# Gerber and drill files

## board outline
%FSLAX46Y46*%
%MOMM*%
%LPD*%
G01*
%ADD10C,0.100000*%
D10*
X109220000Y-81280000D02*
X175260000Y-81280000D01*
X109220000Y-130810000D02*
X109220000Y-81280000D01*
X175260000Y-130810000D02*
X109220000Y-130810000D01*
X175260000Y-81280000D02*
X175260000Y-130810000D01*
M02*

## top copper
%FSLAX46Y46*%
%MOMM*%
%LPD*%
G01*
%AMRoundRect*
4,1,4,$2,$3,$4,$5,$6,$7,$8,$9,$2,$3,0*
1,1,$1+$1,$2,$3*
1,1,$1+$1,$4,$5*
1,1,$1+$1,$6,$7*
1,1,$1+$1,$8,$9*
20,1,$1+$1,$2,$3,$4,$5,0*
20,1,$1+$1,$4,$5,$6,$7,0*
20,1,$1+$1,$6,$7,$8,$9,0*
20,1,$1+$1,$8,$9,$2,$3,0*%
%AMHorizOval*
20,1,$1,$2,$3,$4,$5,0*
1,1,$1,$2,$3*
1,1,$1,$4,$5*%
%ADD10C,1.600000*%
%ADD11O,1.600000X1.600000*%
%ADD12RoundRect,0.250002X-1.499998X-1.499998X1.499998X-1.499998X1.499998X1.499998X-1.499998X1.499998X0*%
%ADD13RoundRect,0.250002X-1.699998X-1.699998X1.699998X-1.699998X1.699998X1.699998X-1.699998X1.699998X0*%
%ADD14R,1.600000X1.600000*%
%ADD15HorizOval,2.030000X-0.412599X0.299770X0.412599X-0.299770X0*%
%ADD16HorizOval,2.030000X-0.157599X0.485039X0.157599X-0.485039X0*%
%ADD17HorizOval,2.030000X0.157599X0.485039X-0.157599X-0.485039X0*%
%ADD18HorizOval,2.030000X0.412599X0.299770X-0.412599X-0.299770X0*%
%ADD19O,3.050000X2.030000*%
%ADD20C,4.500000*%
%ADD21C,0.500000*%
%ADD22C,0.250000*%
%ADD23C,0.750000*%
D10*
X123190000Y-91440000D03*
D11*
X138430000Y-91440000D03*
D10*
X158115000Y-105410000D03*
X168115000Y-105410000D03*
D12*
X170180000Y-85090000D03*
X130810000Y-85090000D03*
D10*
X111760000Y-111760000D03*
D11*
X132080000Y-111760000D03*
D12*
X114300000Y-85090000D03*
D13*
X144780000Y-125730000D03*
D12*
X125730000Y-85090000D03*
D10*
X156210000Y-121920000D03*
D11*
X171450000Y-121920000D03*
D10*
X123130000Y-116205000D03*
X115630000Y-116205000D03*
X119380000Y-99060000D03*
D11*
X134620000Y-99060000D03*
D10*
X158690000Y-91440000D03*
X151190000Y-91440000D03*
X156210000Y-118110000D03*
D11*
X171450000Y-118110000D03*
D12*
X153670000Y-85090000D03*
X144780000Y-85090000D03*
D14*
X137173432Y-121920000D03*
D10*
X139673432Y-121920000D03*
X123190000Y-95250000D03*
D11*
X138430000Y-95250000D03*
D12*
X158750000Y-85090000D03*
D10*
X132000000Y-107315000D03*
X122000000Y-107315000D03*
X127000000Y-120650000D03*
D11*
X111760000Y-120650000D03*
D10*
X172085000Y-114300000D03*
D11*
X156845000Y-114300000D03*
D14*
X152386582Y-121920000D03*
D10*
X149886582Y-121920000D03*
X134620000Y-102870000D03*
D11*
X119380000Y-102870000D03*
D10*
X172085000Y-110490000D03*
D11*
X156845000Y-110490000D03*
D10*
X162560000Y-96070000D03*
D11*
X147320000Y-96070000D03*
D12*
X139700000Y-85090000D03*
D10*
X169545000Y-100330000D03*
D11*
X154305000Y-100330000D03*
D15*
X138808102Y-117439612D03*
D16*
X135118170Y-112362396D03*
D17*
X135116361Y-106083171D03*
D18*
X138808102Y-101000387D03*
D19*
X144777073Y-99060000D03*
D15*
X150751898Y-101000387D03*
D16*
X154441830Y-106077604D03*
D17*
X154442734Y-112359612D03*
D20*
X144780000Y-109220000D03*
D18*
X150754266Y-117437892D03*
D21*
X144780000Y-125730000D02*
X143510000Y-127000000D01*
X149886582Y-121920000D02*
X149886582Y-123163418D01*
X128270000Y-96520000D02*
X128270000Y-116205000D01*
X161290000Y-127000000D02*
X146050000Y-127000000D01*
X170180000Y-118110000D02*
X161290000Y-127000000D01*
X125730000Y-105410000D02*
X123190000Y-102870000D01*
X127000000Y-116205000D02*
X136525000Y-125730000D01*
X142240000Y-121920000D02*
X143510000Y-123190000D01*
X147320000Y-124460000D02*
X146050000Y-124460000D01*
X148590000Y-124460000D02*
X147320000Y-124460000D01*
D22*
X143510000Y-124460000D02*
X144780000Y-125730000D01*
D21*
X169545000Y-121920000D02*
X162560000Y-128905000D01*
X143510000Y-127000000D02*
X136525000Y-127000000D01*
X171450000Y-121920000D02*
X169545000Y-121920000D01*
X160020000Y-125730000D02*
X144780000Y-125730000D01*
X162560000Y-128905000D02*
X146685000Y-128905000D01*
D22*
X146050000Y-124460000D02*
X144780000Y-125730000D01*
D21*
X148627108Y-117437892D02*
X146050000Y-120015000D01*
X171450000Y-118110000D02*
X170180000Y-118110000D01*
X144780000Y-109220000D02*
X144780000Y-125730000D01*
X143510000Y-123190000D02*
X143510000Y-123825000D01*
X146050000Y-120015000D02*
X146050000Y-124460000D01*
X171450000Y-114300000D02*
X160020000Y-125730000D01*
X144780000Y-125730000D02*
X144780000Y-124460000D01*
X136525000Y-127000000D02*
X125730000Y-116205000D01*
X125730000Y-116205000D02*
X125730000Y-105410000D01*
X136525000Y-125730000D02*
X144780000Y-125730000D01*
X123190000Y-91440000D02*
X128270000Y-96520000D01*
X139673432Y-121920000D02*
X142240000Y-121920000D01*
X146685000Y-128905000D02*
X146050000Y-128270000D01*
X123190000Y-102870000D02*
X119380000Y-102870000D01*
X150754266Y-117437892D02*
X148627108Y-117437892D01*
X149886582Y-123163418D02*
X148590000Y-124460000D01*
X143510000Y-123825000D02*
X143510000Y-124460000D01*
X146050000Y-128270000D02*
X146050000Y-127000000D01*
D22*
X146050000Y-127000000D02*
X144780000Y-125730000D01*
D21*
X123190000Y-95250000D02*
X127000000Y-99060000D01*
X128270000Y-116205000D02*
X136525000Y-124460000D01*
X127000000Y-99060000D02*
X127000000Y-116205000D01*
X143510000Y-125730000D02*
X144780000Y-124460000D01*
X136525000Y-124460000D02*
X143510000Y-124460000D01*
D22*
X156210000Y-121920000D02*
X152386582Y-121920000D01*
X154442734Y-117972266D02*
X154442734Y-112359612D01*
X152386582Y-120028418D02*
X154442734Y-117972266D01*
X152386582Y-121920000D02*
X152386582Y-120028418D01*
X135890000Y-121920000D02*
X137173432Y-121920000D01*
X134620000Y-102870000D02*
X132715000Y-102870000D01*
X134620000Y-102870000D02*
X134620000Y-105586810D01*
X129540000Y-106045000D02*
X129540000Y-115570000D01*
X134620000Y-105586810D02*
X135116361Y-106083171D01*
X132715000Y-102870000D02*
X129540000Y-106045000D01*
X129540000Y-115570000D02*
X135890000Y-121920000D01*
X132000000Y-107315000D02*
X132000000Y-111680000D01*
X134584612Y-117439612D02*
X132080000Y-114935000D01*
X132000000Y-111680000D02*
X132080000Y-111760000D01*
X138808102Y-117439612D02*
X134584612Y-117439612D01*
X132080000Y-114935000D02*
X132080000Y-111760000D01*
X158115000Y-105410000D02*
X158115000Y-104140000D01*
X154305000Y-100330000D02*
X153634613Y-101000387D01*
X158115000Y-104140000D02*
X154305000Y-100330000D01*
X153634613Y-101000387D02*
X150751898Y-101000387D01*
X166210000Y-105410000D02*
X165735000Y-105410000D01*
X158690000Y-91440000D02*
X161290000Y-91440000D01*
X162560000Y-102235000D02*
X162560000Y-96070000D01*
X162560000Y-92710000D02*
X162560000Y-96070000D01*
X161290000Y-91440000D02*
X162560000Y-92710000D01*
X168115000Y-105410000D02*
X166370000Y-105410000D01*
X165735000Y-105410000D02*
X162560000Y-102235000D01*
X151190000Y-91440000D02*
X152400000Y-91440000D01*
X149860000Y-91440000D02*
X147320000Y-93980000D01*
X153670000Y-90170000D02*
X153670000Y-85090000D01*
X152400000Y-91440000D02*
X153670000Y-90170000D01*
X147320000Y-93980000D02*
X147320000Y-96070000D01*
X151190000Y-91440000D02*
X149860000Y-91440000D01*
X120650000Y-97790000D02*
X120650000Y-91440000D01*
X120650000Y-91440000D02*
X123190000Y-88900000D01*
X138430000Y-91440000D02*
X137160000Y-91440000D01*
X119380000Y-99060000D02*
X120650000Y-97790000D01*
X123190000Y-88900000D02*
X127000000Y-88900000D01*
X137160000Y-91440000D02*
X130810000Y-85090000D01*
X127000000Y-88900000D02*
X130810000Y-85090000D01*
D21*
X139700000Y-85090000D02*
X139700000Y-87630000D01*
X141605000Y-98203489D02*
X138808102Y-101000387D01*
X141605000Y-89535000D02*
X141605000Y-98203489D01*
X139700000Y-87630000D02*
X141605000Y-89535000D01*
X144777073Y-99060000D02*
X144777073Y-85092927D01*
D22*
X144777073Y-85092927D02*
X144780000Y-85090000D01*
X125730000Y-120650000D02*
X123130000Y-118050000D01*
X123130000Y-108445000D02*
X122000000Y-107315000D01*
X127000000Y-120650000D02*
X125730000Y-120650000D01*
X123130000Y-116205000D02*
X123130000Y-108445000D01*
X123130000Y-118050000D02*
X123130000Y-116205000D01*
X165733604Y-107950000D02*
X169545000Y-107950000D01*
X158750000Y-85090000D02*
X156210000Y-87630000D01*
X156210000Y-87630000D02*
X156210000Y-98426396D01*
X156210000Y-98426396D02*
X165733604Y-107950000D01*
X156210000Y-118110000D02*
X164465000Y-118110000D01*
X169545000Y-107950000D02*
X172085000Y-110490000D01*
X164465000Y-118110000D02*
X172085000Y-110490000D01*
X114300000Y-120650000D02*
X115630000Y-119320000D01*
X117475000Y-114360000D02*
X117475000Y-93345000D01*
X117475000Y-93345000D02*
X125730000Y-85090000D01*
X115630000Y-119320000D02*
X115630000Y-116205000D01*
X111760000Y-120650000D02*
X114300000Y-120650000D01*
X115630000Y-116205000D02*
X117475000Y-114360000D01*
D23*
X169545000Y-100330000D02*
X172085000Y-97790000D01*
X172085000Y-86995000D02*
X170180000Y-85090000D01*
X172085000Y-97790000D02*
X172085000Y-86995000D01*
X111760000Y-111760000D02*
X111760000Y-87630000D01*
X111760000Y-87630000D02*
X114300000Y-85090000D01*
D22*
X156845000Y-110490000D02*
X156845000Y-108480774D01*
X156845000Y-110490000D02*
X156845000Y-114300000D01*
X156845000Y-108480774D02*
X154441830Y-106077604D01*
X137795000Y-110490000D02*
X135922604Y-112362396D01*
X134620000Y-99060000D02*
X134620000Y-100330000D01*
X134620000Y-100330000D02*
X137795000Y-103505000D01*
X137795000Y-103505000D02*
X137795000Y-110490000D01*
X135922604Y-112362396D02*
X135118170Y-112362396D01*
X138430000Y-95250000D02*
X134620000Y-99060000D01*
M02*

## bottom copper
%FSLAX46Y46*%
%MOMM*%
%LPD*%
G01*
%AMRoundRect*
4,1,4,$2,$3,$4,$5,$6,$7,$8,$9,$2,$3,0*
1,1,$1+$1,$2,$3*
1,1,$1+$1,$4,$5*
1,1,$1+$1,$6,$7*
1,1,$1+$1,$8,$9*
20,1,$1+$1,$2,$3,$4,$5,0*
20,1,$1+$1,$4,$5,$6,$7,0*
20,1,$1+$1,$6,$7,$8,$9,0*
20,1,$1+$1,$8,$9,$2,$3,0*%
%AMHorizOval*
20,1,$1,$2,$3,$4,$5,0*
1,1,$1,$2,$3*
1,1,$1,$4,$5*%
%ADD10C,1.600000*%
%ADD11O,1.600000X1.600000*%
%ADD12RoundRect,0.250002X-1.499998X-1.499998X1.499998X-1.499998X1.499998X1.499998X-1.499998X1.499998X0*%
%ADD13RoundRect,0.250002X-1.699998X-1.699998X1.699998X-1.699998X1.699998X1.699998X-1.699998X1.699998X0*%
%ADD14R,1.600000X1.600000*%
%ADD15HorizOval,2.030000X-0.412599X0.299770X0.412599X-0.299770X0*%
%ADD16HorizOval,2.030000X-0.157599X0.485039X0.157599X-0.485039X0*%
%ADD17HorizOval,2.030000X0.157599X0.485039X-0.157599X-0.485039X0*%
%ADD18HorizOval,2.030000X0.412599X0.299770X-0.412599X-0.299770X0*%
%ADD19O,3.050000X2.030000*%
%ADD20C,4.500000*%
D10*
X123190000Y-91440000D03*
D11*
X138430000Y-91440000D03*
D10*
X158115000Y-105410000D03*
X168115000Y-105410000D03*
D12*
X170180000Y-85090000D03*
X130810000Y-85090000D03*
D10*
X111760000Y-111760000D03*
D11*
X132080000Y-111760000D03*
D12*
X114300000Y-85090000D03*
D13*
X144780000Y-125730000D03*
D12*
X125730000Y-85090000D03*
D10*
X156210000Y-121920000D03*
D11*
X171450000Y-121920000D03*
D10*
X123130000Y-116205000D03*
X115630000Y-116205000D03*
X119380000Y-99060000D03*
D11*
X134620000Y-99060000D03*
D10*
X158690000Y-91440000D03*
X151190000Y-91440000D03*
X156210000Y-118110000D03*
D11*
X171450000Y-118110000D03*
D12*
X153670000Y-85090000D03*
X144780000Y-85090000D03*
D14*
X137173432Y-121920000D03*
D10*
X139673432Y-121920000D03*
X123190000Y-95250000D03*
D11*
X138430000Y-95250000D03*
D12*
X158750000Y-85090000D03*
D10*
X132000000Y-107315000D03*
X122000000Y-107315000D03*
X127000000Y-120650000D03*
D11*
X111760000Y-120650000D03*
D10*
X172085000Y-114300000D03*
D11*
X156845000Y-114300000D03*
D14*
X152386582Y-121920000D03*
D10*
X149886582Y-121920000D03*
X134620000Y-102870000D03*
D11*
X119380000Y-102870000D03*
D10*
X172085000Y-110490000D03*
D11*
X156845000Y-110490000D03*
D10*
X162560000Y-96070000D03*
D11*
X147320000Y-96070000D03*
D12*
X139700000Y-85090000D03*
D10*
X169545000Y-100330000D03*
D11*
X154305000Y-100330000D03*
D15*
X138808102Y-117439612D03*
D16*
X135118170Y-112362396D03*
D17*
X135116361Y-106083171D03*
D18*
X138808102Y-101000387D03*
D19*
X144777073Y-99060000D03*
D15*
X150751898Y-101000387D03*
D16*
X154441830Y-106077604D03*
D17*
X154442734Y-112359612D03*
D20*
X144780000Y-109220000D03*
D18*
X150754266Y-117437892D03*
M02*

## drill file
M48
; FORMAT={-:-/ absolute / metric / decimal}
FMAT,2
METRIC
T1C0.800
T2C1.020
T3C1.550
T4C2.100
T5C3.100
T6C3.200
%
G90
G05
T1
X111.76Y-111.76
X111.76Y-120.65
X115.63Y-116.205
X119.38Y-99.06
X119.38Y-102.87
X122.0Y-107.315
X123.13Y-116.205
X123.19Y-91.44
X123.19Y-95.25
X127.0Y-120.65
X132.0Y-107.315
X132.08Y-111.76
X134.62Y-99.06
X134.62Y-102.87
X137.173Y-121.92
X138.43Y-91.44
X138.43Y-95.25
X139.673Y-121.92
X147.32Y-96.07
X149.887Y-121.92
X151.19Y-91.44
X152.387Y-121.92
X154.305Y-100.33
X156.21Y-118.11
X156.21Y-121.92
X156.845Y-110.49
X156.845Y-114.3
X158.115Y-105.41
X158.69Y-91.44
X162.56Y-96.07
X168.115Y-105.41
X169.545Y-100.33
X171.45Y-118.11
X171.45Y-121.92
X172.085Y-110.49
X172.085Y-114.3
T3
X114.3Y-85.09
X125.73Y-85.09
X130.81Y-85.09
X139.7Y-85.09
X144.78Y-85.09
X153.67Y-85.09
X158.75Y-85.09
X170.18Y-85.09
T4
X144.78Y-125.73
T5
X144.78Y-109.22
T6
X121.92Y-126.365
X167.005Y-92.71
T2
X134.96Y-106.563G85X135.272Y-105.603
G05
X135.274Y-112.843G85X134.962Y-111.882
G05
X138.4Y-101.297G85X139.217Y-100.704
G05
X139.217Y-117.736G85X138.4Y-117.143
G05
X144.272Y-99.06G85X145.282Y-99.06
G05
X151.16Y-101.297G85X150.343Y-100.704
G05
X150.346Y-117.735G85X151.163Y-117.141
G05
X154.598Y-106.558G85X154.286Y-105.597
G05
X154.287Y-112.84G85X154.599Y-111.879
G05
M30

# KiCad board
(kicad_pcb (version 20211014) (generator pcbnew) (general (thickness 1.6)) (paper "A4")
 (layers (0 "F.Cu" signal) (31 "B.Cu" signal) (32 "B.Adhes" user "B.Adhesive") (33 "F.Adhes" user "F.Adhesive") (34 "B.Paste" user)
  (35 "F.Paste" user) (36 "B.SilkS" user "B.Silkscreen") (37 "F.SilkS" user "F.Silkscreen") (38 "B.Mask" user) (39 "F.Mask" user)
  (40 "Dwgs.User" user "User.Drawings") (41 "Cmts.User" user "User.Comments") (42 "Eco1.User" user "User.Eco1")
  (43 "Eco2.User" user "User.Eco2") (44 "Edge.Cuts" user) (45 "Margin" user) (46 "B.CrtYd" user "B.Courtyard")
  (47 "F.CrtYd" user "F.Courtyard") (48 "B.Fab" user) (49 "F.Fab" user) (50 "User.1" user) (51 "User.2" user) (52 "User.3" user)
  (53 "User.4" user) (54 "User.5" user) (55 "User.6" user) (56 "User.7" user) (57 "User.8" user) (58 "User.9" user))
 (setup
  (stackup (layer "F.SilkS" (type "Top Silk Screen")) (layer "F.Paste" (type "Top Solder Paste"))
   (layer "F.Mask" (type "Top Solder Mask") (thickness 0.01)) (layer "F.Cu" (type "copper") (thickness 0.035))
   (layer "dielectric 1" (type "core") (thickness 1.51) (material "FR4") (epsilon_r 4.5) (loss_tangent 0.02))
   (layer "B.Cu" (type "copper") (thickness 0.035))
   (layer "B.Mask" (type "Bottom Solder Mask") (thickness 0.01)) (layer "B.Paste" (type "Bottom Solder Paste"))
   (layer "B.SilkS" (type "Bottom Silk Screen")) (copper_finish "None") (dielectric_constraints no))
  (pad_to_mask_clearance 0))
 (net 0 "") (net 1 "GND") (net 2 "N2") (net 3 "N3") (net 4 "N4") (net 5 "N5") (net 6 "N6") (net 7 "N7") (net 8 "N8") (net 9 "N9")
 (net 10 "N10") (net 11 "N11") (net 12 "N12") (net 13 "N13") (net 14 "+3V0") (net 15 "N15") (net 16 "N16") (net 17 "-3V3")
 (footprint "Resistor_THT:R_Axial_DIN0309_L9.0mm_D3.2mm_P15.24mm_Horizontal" (layer "F.Cu") (at 123.19 91.44)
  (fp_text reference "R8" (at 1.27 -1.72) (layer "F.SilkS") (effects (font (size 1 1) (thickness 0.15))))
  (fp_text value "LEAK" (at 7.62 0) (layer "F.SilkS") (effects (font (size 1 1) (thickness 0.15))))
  (pad "1" thru_hole circle (at 0 0) (size 1.6 1.6) (drill 0.8) (layers *.Cu *.Mask) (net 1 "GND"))
  (pad "2" thru_hole oval (at 15.24 0) (size 1.6 1.6) (drill 0.8) (layers *.Cu *.Mask) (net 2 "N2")))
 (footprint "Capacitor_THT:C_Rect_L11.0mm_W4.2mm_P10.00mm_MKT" (layer "F.Cu") (at 158.115 105.41)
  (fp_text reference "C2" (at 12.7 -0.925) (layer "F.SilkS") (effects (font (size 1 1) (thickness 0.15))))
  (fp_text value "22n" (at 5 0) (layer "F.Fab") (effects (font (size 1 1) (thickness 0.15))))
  (pad "1" thru_hole circle (at 0 0) (size 1.6 1.6) (drill 0.8) (layers *.Cu *.Mask) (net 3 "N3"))
  (pad "2" thru_hole circle (at 10 0) (size 1.6 1.6) (drill 0.8) (layers *.Cu *.Mask) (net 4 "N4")))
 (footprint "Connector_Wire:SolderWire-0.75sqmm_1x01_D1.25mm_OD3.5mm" (layer "F.Cu") (at 170.18 85.09)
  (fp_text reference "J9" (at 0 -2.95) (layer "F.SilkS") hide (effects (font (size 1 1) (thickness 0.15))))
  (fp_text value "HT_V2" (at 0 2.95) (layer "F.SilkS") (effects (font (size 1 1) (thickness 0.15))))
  (pad "1" thru_hole roundrect (at 0 0) (size 3.5 3.5) (drill 1.55) (layers *.Cu *.Mask) (roundrect_rratio 0.07142914286) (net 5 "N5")))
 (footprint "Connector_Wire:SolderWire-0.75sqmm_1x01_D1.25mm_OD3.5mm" (layer "F.Cu") (at 130.81 85.09)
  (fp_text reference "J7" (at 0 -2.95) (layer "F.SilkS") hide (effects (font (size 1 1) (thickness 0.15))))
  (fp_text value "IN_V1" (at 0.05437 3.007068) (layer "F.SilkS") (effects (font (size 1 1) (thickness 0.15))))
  (pad "1" thru_hole roundrect (at 0 0) (size 3.5 3.5) (drill 1.55) (layers *.Cu *.Mask) (roundrect_rratio 0.07142914286) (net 2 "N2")))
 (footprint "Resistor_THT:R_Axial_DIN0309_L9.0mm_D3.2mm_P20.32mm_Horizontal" (layer "F.Cu") (at 111.76 111.76)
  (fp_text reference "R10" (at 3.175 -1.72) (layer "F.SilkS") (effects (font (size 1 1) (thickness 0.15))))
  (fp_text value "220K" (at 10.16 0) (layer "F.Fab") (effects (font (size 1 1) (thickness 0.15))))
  (pad "1" thru_hole circle (at 0 0) (size 1.6 1.6) (drill 0.8) (layers *.Cu *.Mask) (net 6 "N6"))
  (pad "2" thru_hole oval (at 20.32 0) (size 1.6 1.6) (drill 0.8) (layers *.Cu *.Mask) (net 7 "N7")))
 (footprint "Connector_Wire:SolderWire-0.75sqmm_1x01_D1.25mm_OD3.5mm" (layer "F.Cu") (at 114.3 85.09)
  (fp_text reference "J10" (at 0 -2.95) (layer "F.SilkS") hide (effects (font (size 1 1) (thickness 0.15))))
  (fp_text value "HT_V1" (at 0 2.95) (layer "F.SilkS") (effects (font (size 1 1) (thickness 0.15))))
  (pad "1" thru_hole roundrect (at 0 0) (size 3.5 3.5) (drill 1.55) (layers *.Cu *.Mask) (roundrect_rratio 0.07142914286) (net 6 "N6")))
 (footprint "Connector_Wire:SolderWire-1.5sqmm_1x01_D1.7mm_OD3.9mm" (layer "F.Cu") (at 144.78 125.73)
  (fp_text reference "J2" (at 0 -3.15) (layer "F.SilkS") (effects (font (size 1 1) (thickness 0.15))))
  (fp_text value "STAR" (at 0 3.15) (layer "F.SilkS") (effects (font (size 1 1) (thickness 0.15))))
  (pad "1" thru_hole roundrect (at 0 0) (size 3.9 3.9) (drill 2.1) (layers *.Cu *.Mask) (roundrect_rratio 0.06410307692) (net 1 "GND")))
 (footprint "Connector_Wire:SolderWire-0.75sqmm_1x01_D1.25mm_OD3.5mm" (layer "F.Cu") (at 125.73 85.09)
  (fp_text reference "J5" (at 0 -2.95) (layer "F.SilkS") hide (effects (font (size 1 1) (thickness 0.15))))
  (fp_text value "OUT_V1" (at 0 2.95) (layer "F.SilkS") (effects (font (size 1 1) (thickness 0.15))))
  (pad "1" thru_hole roundrect (at 0 0) (size 3.5 3.5) (drill 1.55) (layers *.Cu *.Mask) (roundrect_rratio 0.07142914286) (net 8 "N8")))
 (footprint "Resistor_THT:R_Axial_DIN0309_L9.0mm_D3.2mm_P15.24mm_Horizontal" (layer "F.Cu") (at 156.21 121.92)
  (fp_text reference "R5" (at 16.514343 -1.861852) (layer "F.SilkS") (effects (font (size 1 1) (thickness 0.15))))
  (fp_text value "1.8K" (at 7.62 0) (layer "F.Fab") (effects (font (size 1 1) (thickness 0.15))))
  (pad "1" thru_hole circle (at 0 0) (size 1.6 1.6) (drill 0.8) (layers *.Cu *.Mask) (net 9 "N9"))
  (pad "2" thru_hole oval (at 15.24 0) (size 1.6 1.6) (drill 0.8) (layers *.Cu *.Mask) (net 1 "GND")))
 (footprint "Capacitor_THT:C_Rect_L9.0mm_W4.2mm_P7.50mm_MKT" (layer "F.Cu") (at 123.13 116.205 180)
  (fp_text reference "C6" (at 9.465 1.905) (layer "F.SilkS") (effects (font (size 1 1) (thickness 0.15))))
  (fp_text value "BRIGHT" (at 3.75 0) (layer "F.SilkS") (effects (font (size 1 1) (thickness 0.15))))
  (pad "1" thru_hole circle (at 0 0 180) (size 1.6 1.6) (drill 0.8) (layers *.Cu *.Mask) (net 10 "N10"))
  (pad "2" thru_hole circle (at 7.5 0 180) (size 1.6 1.6) (drill 0.8) (layers *.Cu *.Mask) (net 8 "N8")))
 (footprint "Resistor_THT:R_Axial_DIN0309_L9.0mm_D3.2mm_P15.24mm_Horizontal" (layer "F.Cu") (at 119.38 99.06)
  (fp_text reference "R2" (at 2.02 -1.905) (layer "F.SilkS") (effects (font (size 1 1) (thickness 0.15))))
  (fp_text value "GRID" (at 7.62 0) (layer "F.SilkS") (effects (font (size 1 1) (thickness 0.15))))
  (pad "1" thru_hole circle (at 0 0) (size 1.6 1.6) (drill 0.8) (layers *.Cu *.Mask) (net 2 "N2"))
  (pad "2" thru_hole oval (at 15.24 0) (size 1.6 1.6) (drill 0.8) (layers *.Cu *.Mask) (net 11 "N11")))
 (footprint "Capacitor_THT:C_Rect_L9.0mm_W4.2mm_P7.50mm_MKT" (layer "F.Cu") (at 158.69 91.44 180)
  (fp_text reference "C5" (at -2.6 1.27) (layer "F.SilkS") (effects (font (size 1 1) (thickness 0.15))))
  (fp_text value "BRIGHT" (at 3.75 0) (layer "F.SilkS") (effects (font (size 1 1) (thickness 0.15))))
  (pad "1" thru_hole circle (at 0 0 180) (size 1.6 1.6) (drill 0.8) (layers *.Cu *.Mask) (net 4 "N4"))
  (pad "2" thru_hole circle (at 7.5 0 180) (size 1.6 1.6) (drill 0.8) (layers *.Cu *.Mask) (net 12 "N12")))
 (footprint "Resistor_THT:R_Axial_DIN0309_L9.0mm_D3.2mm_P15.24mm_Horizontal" (layer "F.Cu") (at 156.21 118.11)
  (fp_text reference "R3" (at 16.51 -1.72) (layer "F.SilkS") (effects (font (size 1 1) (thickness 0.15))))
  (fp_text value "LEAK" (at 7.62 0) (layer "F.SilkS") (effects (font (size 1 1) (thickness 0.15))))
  (pad "1" thru_hole circle (at 0 0) (size 1.6 1.6) (drill 0.8) (layers *.Cu *.Mask) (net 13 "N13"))
  (pad "2" thru_hole oval (at 15.24 0) (size 1.6 1.6) (drill 0.8) (layers *.Cu *.Mask) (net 1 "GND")))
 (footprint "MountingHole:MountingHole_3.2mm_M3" (layer "F.Cu") (at 167.005 92.71)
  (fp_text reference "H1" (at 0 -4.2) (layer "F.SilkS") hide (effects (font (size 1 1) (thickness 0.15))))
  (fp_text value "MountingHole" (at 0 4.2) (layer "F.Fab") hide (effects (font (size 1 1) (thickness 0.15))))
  (pad "" np_thru_hole circle (at 0 0) (size 3.2 3.2) (drill 3.2) (layers *.Cu *.Mask)))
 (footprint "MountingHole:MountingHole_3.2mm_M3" (layer "F.Cu") (at 121.92 126.365)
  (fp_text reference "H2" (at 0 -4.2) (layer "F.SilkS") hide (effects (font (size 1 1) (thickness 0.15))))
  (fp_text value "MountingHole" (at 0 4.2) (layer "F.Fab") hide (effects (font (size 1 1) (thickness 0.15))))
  (pad "" np_thru_hole circle (at 0 0) (size 3.2 3.2) (drill 3.2) (layers *.Cu *.Mask)))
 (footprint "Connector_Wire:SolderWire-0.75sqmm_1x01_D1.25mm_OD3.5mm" (layer "F.Cu") (at 153.67 85.09)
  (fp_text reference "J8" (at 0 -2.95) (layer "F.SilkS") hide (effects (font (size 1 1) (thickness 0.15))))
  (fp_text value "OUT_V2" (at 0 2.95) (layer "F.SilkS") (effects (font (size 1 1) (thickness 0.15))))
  (pad "1" thru_hole roundrect (at 0 0) (size 3.5 3.5) (drill 1.55) (layers *.Cu *.Mask) (roundrect_rratio 0.07142914286) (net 12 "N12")))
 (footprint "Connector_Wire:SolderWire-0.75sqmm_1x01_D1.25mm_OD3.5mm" (layer "F.Cu") (at 144.78 85.09)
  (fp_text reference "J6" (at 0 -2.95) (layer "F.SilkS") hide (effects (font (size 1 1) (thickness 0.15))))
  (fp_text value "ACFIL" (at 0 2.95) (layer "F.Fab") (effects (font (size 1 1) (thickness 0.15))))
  (pad "1" thru_hole roundrect (at 0 0) (size 3.5 3.5) (drill 1.55) (layers *.Cu *.Mask) (roundrect_rratio 0.07142914286) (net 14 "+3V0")))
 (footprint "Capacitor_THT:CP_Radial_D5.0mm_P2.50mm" (layer "F.Cu") (at 137.173432 121.92)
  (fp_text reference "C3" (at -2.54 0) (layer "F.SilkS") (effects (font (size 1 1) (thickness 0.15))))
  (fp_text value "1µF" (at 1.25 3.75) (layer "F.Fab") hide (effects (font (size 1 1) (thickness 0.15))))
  (pad "1" thru_hole rect (at 0 0) (size 1.6 1.6) (drill 0.8) (layers *.Cu *.Mask) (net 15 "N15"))
  (pad "2" thru_hole circle (at 2.5 0) (size 1.6 1.6) (drill 0.8) (layers *.Cu *.Mask) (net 1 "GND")))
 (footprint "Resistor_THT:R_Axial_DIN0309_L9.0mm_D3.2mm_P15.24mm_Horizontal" (layer "F.Cu") (at 123.19 95.25)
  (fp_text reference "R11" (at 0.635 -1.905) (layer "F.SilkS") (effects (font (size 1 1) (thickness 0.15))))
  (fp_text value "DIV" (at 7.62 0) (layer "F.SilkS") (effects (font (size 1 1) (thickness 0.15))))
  (pad "1" thru_hole circle (at 0 0) (size 1.6 1.6) (drill 0.8) (layers *.Cu *.Mask) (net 1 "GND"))
  (pad "2" thru_hole oval (at 15.24 0) (size 1.6 1.6) (drill 0.8) (layers *.Cu *.Mask) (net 11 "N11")))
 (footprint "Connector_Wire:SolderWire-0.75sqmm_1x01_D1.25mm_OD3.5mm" (layer "F.Cu") (at 158.75 85.09)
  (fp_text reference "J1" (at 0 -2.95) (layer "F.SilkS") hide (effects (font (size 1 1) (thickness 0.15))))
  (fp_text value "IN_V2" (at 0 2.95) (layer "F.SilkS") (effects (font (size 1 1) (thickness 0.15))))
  (pad "1" thru_hole roundrect (at 0 0) (size 3.5 3.5) (drill 1.55) (layers *.Cu *.Mask) (roundrect_rratio 0.07142914286) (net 13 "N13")))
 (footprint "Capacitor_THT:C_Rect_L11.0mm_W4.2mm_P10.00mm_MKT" (layer "F.Cu") (at 132 107.315 180)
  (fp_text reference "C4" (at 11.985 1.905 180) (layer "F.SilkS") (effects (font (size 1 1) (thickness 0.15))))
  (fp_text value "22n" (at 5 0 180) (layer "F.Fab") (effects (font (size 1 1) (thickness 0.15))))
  (pad "1" thru_hole circle (at 0 0 180) (size 1.6 1.6) (drill 0.8) (layers *.Cu *.Mask) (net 7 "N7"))
  (pad "2" thru_hole circle (at 10 0 180) (size 1.6 1.6) (drill 0.8) (layers *.Cu *.Mask) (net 10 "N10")))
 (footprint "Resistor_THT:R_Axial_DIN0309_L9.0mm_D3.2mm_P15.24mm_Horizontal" (layer "F.Cu") (at 127 120.65 180)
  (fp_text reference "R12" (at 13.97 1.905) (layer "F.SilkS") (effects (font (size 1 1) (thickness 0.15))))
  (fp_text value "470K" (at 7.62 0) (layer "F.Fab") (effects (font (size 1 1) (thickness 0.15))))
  (pad "1" thru_hole circle (at 0 0 180) (size 1.6 1.6) (drill 0.8) (layers *.Cu *.Mask) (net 10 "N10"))
  (pad "2" thru_hole oval (at 15.24 0 180) (size 1.6 1.6) (drill 0.8) (layers *.Cu *.Mask) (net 8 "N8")))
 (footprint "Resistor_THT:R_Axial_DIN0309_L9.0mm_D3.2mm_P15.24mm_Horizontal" (layer "F.Cu") (at 172.085 114.3 180)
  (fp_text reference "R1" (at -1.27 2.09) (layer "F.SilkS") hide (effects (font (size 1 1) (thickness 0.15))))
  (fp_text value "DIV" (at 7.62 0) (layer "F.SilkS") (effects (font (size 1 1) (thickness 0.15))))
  (pad "1" thru_hole circle (at 0 0 180) (size 1.6 1.6) (drill 0.8) (layers *.Cu *.Mask) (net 1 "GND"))
  (pad "2" thru_hole oval (at 15.24 0 180) (size 1.6 1.6) (drill 0.8) (layers *.Cu *.Mask) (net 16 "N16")))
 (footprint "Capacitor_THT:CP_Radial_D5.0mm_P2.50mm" (layer "F.Cu") (at 152.386582 121.92 180)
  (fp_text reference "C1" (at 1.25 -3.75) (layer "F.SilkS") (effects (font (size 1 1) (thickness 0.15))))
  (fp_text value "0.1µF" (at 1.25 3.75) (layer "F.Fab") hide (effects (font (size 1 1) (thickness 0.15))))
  (pad "1" thru_hole rect (at 0 0 180) (size 1.6 1.6) (drill 0.8) (layers *.Cu *.Mask) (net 9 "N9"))
  (pad "2" thru_hole circle (at 2.5 0 180) (size 1.6 1.6) (drill 0.8) (layers *.Cu *.Mask) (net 1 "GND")))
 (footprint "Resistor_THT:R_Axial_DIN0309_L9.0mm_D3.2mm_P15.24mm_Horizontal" (layer "F.Cu") (at 134.62 102.87 180)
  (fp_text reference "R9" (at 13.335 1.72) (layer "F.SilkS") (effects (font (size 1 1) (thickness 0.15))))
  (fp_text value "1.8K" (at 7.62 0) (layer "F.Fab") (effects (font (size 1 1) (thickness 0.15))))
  (pad "1" thru_hole circle (at 0 0 180) (size 1.6 1.6) (drill 0.8) (layers *.Cu *.Mask) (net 15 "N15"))
  (pad "2" thru_hole oval (at 15.24 0 180) (size 1.6 1.6) (drill 0.8) (layers *.Cu *.Mask) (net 1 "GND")))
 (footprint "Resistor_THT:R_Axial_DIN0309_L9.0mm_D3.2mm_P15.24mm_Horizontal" (layer "F.Cu") (at 172.085 110.49 180)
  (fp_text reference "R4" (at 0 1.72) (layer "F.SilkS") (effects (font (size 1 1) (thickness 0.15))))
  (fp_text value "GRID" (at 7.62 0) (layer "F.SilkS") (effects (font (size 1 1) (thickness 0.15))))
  (pad "1" thru_hole circle (at 0 0 180) (size 1.6 1.6) (drill 0.8) (layers *.Cu *.Mask) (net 13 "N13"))
  (pad "2" thru_hole oval (at 15.24 0 180) (size 1.6 1.6) (drill 0.8) (layers *.Cu *.Mask) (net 16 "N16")))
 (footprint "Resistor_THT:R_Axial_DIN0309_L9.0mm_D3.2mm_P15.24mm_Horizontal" (layer "F.Cu") (at 162.56 96.07 180)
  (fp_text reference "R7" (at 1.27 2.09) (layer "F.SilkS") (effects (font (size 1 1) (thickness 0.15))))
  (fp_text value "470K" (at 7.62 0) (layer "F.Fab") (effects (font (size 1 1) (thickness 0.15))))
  (pad "1" thru_hole circle (at 0 0 180) (size 1.6 1.6) (drill 0.8) (layers *.Cu *.Mask) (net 4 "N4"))
  (pad "2" thru_hole oval (at 15.24 0 180) (size 1.6 1.6) (drill 0.8) (layers *.Cu *.Mask) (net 12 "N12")))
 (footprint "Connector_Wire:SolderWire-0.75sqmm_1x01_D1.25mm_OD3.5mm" (layer "F.Cu") (at 139.7 85.09)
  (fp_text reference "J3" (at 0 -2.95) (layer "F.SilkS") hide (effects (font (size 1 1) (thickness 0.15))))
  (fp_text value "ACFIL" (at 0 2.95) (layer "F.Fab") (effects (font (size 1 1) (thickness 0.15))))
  (pad "1" thru_hole roundrect (at 0 0) (size 3.5 3.5) (drill 1.55) (layers *.Cu *.Mask) (roundrect_rratio 0.07142914286) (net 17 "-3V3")))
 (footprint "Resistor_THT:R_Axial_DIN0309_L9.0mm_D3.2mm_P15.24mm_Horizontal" (layer "F.Cu") (at 169.545 100.33 180)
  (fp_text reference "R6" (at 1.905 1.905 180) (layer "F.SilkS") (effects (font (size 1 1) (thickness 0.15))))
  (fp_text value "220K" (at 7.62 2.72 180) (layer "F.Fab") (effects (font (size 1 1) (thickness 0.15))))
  (pad "1" thru_hole circle (at 0 0 180) (size 1.6 1.6) (drill 0.8) (layers *.Cu *.Mask) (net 5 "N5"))
  (pad "2" thru_hole oval (at 15.24 0 180) (size 1.6 1.6) (drill 0.8) (layers *.Cu *.Mask) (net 3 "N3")))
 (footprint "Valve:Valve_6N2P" (layer "B.Cu") (at 141.33 113.97 180)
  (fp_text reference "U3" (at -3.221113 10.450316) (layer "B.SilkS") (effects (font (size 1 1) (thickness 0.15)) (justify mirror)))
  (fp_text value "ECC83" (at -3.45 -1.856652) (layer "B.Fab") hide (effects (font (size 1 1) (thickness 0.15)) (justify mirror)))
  (pad "1" thru_hole oval (at 2.521898 -3.469612 234) (size 2.03 3.05) (drill oval 1.02 2.03) (layers *.Cu *.Mask) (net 7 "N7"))
  (pad "2" thru_hole oval (at 6.21183 1.607604 198) (size 2.03 3.05) (drill oval 1.02 2.03) (layers *.Cu *.Mask) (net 11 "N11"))
  (pad "3" thru_hole oval (at 6.213639 7.886829 162) (size 2.03 3.05) (drill oval 1.02 2.03) (layers *.Cu *.Mask) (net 15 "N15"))
  (pad "4" thru_hole oval (at 2.521898 12.969613 126) (size 2.03 3.05) (drill oval 1.02 2.03) (layers *.Cu *.Mask) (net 17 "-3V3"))
  (pad "5" thru_hole oval (at -3.447073 14.91 90) (size 2.03 3.05) (drill oval 1.02 2.03) (layers *.Cu *.Mask) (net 14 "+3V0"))
  (pad "6" thru_hole oval (at -9.421898 12.969613 234) (size 2.03 3.05) (drill oval 1.02 2.03) (layers *.Cu *.Mask) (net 3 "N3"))
  (pad "7" thru_hole oval (at -13.11183 7.892396 198) (size 2.03 3.05) (drill oval 1.02 2.03) (layers *.Cu *.Mask) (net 16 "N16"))
  (pad "8" thru_hole oval (at -13.112734 1.610388 162) (size 2.03 3.05) (drill oval 1.02 2.03) (layers *.Cu *.Mask) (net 9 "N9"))
  (pad "9" thru_hole circle (at -3.45 4.75 180) (size 4.5 4.5) (drill 3.1) (layers *.Cu *.Mask) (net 1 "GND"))
  (pad "9" thru_hole oval (at -9.424266 -3.467892 126) (size 2.03 3.05) (drill oval 1.02 2.03) (layers *.Cu *.Mask) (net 1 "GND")))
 (gr_line (start 109.22 81.28) (end 175.26 81.28) (layer "Edge.Cuts") (width 0.1))
 (gr_line (start 109.22 130.81) (end 109.22 81.28) (layer "Edge.Cuts") (width 0.1))
 (gr_line (start 175.26 130.81) (end 109.22 130.81) (layer "Edge.Cuts") (width 0.1))
 (gr_line (start 175.26 81.28) (end 175.26 130.81) (layer "Edge.Cuts") (width 0.1))
 (segment (start 144.78 125.73) (end 143.51 127) (width 0.5) (layer "F.Cu") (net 1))
 (segment (start 149.886582 121.92) (end 149.886582 123.163418) (width 0.5) (layer "F.Cu") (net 1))
 (segment (start 128.27 96.52) (end 128.27 116.205) (width 0.5) (layer "F.Cu") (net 1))
 (segment (start 161.29 127) (end 146.05 127) (width 0.5) (layer "F.Cu") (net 1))
 (segment (start 170.18 118.11) (end 161.29 127) (width 0.5) (layer "F.Cu") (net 1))
 (segment (start 125.73 105.41) (end 123.19 102.87) (width 0.5) (layer "F.Cu") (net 1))
 (segment (start 127 116.205) (end 136.525 125.73) (width 0.5) (layer "F.Cu") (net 1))
 (segment (start 142.24 121.92) (end 143.51 123.19) (width 0.5) (layer "F.Cu") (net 1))
 (segment (start 147.32 124.46) (end 146.05 124.46) (width 0.5) (layer "F.Cu") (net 1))
 (segment (start 148.59 124.46) (end 147.32 124.46) (width 0.5) (layer "F.Cu") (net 1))
 (segment (start 143.51 124.46) (end 144.78 125.73) (width 0.25) (layer "F.Cu") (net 1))
 (segment (start 169.545 121.92) (end 162.56 128.905) (width 0.5) (layer "F.Cu") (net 1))
 (segment (start 143.51 127) (end 136.525 127) (width 0.5) (layer "F.Cu") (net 1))
 (segment (start 171.45 121.92) (end 169.545 121.92) (width 0.5) (layer "F.Cu") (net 1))
 (segment (start 160.02 125.73) (end 144.78 125.73) (width 0.5) (layer "F.Cu") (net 1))
 (segment (start 162.56 128.905) (end 146.685 128.905) (width 0.5) (layer "F.Cu") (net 1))
 (segment (start 146.05 124.46) (end 144.78 125.73) (width 0.25) (layer "F.Cu") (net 1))
 (segment (start 148.627108 117.437892) (end 146.05 120.015) (width 0.5) (layer "F.Cu") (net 1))
 (segment (start 171.45 118.11) (end 170.18 118.11) (width 0.5) (layer "F.Cu") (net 1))
 (segment (start 144.78 109.22) (end 144.78 125.73) (width 0.5) (layer "F.Cu") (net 1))
 (segment (start 143.51 123.19) (end 143.51 123.825) (width 0.5) (layer "F.Cu") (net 1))
 (segment (start 146.05 120.015) (end 146.05 124.46) (width 0.5) (layer "F.Cu") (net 1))
 (segment (start 171.45 114.3) (end 160.02 125.73) (width 0.5) (layer "F.Cu") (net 1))
 (segment (start 144.78 125.73) (end 144.78 124.46) (width 0.5) (layer "F.Cu") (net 1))
 (segment (start 136.525 127) (end 125.73 116.205) (width 0.5) (layer "F.Cu") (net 1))
 (segment (start 125.73 116.205) (end 125.73 105.41) (width 0.5) (layer "F.Cu") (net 1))
 (segment (start 136.525 125.73) (end 144.78 125.73) (width 0.5) (layer "F.Cu") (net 1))
 (segment (start 123.19 91.44) (end 128.27 96.52) (width 0.5) (layer "F.Cu") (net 1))
 (segment (start 139.673432 121.92) (end 142.24 121.92) (width 0.5) (layer "F.Cu") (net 1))
 (segment (start 146.685 128.905) (end 146.05 128.27) (width 0.5) (layer "F.Cu") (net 1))
 (segment (start 123.19 102.87) (end 119.38 102.87) (width 0.5) (layer "F.Cu") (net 1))
 (segment (start 150.754266 117.437892) (end 148.627108 117.437892) (width 0.5) (layer "F.Cu") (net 1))
 (segment (start 149.886582 123.163418) (end 148.59 124.46) (width 0.5) (layer "F.Cu") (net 1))
 (segment (start 143.51 123.825) (end 143.51 124.46) (width 0.5) (layer "F.Cu") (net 1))
 (segment (start 146.05 128.27) (end 146.05 127) (width 0.5) (layer "F.Cu") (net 1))
 (segment (start 146.05 127) (end 144.78 125.73) (width 0.25) (layer "F.Cu") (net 1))
 (segment (start 123.19 95.25) (end 127 99.06) (width 0.5) (layer "F.Cu") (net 1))
 (segment (start 128.27 116.205) (end 136.525 124.46) (width 0.5) (layer "F.Cu") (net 1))
 (segment (start 127 99.06) (end 127 116.205) (width 0.5) (layer "F.Cu") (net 1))
 (segment (start 143.51 125.73) (end 144.78 124.46) (width 0.5) (layer "F.Cu") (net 1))
 (segment (start 136.525 124.46) (end 143.51 124.46) (width 0.5) (layer "F.Cu") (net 1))
 (segment (start 156.21 121.92) (end 152.386582 121.92) (width 0.25) (layer "F.Cu") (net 9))
 (segment (start 154.442734 117.972266) (end 154.442734 112.359612) (width 0.25) (layer "F.Cu") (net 9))
 (segment (start 152.386582 120.028418) (end 154.442734 117.972266) (width 0.25) (layer "F.Cu") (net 9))
 (segment (start 152.386582 121.92) (end 152.386582 120.028418) (width 0.25) (layer "F.Cu") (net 9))
 (segment (start 135.89 121.92) (end 137.173432 121.92) (width 0.25) (layer "F.Cu") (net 15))
 (segment (start 134.62 102.87) (end 132.715 102.87) (width 0.25) (layer "F.Cu") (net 15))
 (segment (start 134.62 102.87) (end 134.62 105.58681) (width 0.25) (layer "F.Cu") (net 15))
 (segment (start 129.54 106.045) (end 129.54 115.57) (width 0.25) (layer "F.Cu") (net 15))
 (segment (start 134.62 105.58681) (end 135.116361 106.083171) (width 0.25) (layer "F.Cu") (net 15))
 (segment (start 132.715 102.87) (end 129.54 106.045) (width 0.25) (layer "F.Cu") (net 15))
 (segment (start 129.54 115.57) (end 135.89 121.92) (width 0.25) (layer "F.Cu") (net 15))
 (segment (start 132 107.315) (end 132 111.68) (width 0.25) (layer "F.Cu") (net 7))
 (segment (start 134.584612 117.439612) (end 132.08 114.935) (width 0.25) (layer "F.Cu") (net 7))
 (segment (start 132 111.68) (end 132.08 111.76) (width 0.25) (layer "F.Cu") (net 7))
 (segment (start 138.808102 117.439612) (end 134.584612 117.439612) (width 0.25) (layer "F.Cu") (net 7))
 (segment (start 132.08 114.935) (end 132.08 111.76) (width 0.25) (layer "F.Cu") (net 7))
 (segment (start 158.115 105.41) (end 158.115 104.14) (width 0.25) (layer "F.Cu") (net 3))
 (segment (start 154.305 100.33) (end 153.634613 101.000387) (width 0.25) (layer "F.Cu") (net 3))
 (segment (start 158.115 104.14) (end 154.305 100.33) (width 0.25) (layer "F.Cu") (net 3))
 (segment (start 153.634613 101.000387) (end 150.751898 101.000387) (width 0.25) (layer "F.Cu") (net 3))
 (segment (start 166.21 105.41) (end 165.735 105.41) (width 0.25) (layer "F.Cu") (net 4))
 (segment (start 158.69 91.44) (end 161.29 91.44) (width 0.25) (layer "F.Cu") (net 4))
 (segment (start 162.56 102.235) (end 162.56 96.07) (width 0.25) (layer "F.Cu") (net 4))
 (segment (start 162.56 92.71) (end 162.56 96.07) (width 0.25) (layer "F.Cu") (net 4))
 (segment (start 161.29 91.44) (end 162.56 92.71) (width 0.25) (layer "F.Cu") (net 4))
 (segment (start 168.115 105.41) (end 166.37 105.41) (width 0.25) (layer "F.Cu") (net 4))
 (segment (start 165.735 105.41) (end 162.56 102.235) (width 0.25) (layer "F.Cu") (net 4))
 (segment (start 151.19 91.44) (end 152.4 91.44) (width 0.25) (layer "F.Cu") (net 12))
 (segment (start 149.86 91.44) (end 147.32 93.98) (width 0.25) (layer "F.Cu") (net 12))
 (segment (start 153.67 90.17) (end 153.67 85.09) (width 0.25) (layer "F.Cu") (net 12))
 (segment (start 152.4 91.44) (end 153.67 90.17) (width 0.25) (layer "F.Cu") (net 12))
 (segment (start 147.32 93.98) (end 147.32 96.07) (width 0.25) (layer "F.Cu") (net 12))
 (segment (start 151.19 91.44) (end 149.86 91.44) (width 0.25) (layer "F.Cu") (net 12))
 (segment (start 120.65 97.79) (end 120.65 91.44) (width 0.25) (layer "F.Cu") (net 2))
 (segment (start 120.65 91.44) (end 123.19 88.9) (width 0.25) (layer "F.Cu") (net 2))
 (segment (start 138.43 91.44) (end 137.16 91.44) (width 0.25) (layer "F.Cu") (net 2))
 (segment (start 119.38 99.06) (end 120.65 97.79) (width 0.25) (layer "F.Cu") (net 2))
 (segment (start 123.19 88.9) (end 127 88.9) (width 0.25) (layer "F.Cu") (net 2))
 (segment (start 137.16 91.44) (end 130.81 85.09) (width 0.25) (layer "F.Cu") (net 2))
 (segment (start 127 88.9) (end 130.81 85.09) (width 0.25) (layer "F.Cu") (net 2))
 (segment (start 139.7 85.09) (end 139.7 87.63) (width 0.5) (layer "F.Cu") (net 17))
 (segment (start 141.605 98.203489) (end 138.808102 101.000387) (width 0.5) (layer "F.Cu") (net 17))
 (segment (start 141.605 89.535) (end 141.605 98.203489) (width 0.5) (layer "F.Cu") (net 17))
 (segment (start 139.7 87.63) (end 141.605 89.535) (width 0.5) (layer "F.Cu") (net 17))
 (segment (start 144.777073 99.06) (end 144.777073 85.092927) (width 0.5) (layer "F.Cu") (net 14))
 (segment (start 144.777073 85.092927) (end 144.78 85.09) (width 0.25) (layer "F.Cu") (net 14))
 (segment (start 125.73 120.65) (end 123.13 118.05) (width 0.25) (layer "F.Cu") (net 10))
 (segment (start 123.13 108.445) (end 122 107.315) (width 0.25) (layer "F.Cu") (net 10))
 (segment (start 127 120.65) (end 125.73 120.65) (width 0.25) (layer "F.Cu") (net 10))
 (segment (start 123.13 116.205) (end 123.13 108.445) (width 0.25) (layer "F.Cu") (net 10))
 (segment (start 123.13 118.05) (end 123.13 116.205) (width 0.25) (layer "F.Cu") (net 10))
 (segment (start 165.733604 107.95) (end 169.545 107.95) (width 0.25) (layer "F.Cu") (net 13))
 (segment (start 158.75 85.09) (end 156.21 87.63) (width 0.25) (layer "F.Cu") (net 13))
 (segment (start 156.21 87.63) (end 156.21 98.426396) (width 0.25) (layer "F.Cu") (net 13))
 (segment (start 156.21 98.426396) (end 165.733604 107.95) (width 0.25) (layer "F.Cu") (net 13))
 (segment (start 156.21 118.11) (end 164.465 118.11) (width 0.25) (layer "F.Cu") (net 13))
 (segment (start 169.545 107.95) (end 172.085 110.49) (width 0.25) (layer "F.Cu") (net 13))
 (segment (start 164.465 118.11) (end 172.085 110.49) (width 0.25) (layer "F.Cu") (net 13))
 (segment (start 114.3 120.65) (end 115.63 119.32) (width 0.25) (layer "F.Cu") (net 8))
 (segment (start 117.475 114.36) (end 117.475 93.345) (width 0.25) (layer "F.Cu") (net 8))
 (segment (start 117.475 93.345) (end 125.73 85.09) (width 0.25) (layer "F.Cu") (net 8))
 (segment (start 115.63 119.32) (end 115.63 116.205) (width 0.25) (layer "F.Cu") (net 8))
 (segment (start 111.76 120.65) (end 114.3 120.65) (width 0.25) (layer "F.Cu") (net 8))
 (segment (start 115.63 116.205) (end 117.475 114.36) (width 0.25) (layer "F.Cu") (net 8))
 (segment (start 169.545 100.33) (end 172.085 97.79) (width 0.75) (layer "F.Cu") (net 5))
 (segment (start 172.085 86.995) (end 170.18 85.09) (width 0.75) (layer "F.Cu") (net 5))
 (segment (start 172.085 97.79) (end 172.085 86.995) (width 0.75) (layer "F.Cu") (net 5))
 (segment (start 111.76 111.76) (end 111.76 87.63) (width 0.75) (layer "F.Cu") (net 6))
 (segment (start 111.76 87.63) (end 114.3 85.09) (width 0.75) (layer "F.Cu") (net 6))
 (segment (start 156.845 110.49) (end 156.845 108.480774) (width 0.25) (layer "F.Cu") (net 16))
 (segment (start 156.845 110.49) (end 156.845 114.3) (width 0.25) (layer "F.Cu") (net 16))
 (segment (start 156.845 108.480774) (end 154.44183 106.077604) (width 0.25) (layer "F.Cu") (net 16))
 (segment (start 137.795 110.49) (end 135.922604 112.362396) (width 0.25) (layer "F.Cu") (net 11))
 (segment (start 134.62 99.06) (end 134.62 100.33) (width 0.25) (layer "F.Cu") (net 11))
 (segment (start 134.62 100.33) (end 137.795 103.505) (width 0.25) (layer "F.Cu") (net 11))
 (segment (start 137.795 103.505) (end 137.795 110.49) (width 0.25) (layer "F.Cu") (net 11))
 (segment (start 135.922604 112.362396) (end 135.11817 112.362396) (width 0.25) (layer "F.Cu") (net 11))
 (segment (start 138.43 95.25) (end 134.62 99.06) (width 0.25) (layer "F.Cu") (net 11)))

